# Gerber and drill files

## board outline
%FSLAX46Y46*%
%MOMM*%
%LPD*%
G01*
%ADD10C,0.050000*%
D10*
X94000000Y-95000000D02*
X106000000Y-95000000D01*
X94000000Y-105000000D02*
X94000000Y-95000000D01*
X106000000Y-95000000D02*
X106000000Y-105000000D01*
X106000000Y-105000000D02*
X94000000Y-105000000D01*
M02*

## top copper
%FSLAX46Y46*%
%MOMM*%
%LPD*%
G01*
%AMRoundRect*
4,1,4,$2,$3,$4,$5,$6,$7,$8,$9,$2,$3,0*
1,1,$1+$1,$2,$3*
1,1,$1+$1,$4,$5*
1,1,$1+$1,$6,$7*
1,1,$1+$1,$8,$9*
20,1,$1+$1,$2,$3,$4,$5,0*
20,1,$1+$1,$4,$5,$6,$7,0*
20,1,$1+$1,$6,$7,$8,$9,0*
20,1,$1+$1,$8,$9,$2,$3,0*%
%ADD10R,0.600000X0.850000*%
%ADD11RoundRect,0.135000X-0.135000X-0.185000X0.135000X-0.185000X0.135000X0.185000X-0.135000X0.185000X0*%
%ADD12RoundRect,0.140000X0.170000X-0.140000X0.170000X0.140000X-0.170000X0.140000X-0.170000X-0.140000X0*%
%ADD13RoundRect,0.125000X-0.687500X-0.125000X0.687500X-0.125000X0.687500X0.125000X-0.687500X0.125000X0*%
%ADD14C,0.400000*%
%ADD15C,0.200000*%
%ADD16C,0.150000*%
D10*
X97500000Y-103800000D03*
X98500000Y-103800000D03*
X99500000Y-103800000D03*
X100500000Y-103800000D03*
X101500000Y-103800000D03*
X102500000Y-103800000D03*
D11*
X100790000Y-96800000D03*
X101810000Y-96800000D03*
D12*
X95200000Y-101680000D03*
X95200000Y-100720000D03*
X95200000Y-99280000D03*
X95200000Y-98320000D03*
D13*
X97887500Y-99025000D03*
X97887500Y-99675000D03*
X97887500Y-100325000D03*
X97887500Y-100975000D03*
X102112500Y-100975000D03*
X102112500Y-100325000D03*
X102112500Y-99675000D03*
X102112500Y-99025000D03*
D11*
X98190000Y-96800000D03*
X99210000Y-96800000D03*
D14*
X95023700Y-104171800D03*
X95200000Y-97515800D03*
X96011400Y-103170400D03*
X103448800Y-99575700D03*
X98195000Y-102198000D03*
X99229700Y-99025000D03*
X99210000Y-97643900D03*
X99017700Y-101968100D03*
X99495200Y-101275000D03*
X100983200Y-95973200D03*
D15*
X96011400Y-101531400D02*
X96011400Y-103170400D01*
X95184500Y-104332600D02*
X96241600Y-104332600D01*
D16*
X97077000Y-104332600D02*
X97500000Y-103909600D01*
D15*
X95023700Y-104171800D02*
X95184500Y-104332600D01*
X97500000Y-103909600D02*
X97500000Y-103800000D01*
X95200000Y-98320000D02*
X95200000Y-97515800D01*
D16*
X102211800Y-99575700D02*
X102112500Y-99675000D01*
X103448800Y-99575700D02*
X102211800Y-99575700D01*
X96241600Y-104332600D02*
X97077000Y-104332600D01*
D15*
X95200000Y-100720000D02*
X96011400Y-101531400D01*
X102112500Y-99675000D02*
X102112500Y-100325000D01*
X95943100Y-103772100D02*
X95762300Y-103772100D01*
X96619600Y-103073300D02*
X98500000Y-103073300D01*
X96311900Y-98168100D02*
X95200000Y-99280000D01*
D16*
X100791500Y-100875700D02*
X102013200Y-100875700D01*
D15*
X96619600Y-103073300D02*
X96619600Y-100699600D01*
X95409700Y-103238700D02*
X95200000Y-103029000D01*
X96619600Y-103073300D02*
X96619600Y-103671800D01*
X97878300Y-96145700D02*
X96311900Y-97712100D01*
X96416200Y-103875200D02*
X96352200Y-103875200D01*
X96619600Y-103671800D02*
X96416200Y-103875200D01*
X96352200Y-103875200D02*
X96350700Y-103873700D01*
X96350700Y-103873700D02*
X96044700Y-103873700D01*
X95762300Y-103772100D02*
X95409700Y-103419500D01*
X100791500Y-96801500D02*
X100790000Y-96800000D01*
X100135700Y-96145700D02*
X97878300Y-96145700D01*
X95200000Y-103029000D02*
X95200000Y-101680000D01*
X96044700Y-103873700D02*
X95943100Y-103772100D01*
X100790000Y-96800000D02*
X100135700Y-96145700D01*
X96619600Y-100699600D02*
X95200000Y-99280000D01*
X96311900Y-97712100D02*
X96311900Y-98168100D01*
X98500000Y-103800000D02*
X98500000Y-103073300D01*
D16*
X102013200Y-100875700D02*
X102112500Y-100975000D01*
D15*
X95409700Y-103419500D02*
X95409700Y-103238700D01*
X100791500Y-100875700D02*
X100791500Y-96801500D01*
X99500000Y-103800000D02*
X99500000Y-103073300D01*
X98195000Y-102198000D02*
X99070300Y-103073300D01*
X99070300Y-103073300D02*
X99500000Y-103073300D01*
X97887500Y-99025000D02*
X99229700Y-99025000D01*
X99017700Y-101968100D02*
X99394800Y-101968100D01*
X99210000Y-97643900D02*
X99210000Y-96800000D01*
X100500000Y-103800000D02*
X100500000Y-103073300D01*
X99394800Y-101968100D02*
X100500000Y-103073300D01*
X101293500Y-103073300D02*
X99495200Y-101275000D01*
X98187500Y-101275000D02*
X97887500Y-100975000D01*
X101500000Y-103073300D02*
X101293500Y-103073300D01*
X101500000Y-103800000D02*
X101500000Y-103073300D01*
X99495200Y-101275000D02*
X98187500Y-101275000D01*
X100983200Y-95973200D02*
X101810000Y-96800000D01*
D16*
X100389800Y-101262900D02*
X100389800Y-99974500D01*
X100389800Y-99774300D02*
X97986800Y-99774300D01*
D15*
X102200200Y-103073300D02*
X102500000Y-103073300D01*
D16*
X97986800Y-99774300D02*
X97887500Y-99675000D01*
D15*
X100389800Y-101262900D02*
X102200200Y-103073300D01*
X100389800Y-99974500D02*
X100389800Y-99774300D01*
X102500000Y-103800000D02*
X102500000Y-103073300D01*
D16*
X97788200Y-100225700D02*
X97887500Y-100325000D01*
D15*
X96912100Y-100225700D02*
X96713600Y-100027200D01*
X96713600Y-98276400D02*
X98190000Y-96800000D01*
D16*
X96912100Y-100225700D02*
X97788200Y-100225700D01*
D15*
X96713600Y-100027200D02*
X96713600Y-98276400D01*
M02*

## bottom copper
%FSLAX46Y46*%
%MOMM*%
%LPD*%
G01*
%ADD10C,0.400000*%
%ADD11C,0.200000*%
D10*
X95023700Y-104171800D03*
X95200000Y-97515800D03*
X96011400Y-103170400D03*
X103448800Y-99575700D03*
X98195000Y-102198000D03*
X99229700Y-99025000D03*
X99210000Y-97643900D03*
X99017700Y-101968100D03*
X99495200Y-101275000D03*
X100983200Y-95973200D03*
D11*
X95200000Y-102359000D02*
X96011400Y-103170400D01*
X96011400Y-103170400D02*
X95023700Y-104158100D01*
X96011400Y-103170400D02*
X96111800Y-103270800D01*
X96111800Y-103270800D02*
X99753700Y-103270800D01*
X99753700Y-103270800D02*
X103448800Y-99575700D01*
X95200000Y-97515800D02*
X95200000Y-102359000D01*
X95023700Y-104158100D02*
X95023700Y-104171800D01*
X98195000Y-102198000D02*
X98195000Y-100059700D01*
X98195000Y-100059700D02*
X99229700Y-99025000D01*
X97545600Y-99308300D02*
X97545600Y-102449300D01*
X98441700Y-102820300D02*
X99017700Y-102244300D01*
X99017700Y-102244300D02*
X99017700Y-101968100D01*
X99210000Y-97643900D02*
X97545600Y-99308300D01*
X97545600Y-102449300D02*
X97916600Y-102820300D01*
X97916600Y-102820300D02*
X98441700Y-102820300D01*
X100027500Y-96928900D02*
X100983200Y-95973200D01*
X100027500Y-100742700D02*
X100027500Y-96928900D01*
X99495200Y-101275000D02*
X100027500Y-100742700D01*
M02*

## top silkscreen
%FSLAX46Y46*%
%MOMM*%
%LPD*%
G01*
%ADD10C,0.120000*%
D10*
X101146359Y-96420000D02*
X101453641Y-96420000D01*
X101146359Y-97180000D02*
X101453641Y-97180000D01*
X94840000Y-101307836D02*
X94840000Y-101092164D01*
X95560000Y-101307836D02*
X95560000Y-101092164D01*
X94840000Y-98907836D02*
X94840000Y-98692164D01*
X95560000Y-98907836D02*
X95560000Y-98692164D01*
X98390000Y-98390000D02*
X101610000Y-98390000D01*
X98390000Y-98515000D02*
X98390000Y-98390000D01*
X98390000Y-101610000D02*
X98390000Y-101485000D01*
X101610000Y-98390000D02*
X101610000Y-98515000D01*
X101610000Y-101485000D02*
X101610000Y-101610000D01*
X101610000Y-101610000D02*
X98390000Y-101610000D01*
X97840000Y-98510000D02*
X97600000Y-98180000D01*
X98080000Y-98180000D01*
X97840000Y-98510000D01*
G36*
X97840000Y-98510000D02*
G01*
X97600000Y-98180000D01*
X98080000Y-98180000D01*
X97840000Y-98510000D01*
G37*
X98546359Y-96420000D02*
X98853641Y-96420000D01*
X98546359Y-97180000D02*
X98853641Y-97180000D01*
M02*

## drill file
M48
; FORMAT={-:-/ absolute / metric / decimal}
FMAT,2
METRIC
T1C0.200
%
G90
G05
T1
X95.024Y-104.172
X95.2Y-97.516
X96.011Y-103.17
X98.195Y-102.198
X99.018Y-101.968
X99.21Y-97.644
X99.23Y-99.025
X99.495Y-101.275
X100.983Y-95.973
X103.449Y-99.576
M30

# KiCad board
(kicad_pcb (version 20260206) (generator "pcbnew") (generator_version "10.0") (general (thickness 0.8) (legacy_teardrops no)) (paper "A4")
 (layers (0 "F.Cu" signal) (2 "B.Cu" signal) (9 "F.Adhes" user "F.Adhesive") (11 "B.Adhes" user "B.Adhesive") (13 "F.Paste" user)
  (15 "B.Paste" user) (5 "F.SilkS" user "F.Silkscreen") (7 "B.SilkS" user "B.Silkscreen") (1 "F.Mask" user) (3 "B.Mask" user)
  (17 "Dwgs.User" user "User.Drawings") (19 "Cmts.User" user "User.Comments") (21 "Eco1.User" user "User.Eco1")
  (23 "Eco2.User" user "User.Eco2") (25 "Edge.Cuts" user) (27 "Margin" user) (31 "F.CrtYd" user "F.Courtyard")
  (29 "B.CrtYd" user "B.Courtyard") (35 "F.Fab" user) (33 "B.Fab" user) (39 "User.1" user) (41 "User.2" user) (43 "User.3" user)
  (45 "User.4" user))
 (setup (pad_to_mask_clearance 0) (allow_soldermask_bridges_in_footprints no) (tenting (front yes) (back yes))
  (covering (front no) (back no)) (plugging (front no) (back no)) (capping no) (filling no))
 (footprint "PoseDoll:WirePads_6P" (layer "F.Cu") (at 100 103.8)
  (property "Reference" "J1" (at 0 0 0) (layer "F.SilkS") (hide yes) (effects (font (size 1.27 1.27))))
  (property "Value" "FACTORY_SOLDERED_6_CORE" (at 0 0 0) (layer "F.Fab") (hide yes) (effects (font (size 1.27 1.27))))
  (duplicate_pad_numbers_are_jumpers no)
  (pad "1" smd rect (at -2.5 0) (size 0.6 0.85) (layers "F.Cu" "F.Mask") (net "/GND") (thermal_bridge_angle 45))
  (pad "2" smd rect (at -1.5 0) (size 0.6 0.85) (layers "F.Cu" "F.Mask") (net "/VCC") (thermal_bridge_angle 45))
  (pad "3" smd rect (at -0.5 0) (size 0.6 0.85) (layers "F.Cu" "F.Mask") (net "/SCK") (thermal_bridge_angle 45))
  (pad "4" smd rect (at 0.5 0) (size 0.6 0.85) (layers "F.Cu" "F.Mask") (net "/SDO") (thermal_bridge_angle 45))
  (pad "5" smd rect (at 1.5 0) (size 0.6 0.85) (layers "F.Cu" "F.Mask") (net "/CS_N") (thermal_bridge_angle 45))
  (pad "6" smd rect (at 2.5 0) (size 0.6 0.85) (layers "F.Cu" "F.Mask") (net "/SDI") (thermal_bridge_angle 45)))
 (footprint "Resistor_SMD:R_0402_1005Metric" (layer "F.Cu") (at 101.3 96.8)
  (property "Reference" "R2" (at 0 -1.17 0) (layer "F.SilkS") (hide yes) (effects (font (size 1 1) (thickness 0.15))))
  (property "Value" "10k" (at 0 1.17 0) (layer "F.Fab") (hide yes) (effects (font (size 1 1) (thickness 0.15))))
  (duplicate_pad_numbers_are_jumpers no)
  (fp_line (start -0.153641 -0.38) (end 0.153641 -0.38) (stroke (width 0.12) (type solid)) (layer "F.SilkS"))
  (fp_line (start -0.153641 0.38) (end 0.153641 0.38) (stroke (width 0.12) (type solid)) (layer "F.SilkS"))
  (pad "1" smd roundrect (at -0.51 0) (size 0.54 0.64) (layers "F.Cu" "F.Mask" "F.Paste") (roundrect_rratio 0.25) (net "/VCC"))
  (pad "2" smd roundrect (at 0.51 0) (size 0.54 0.64) (layers "F.Cu" "F.Mask" "F.Paste") (roundrect_rratio 0.25) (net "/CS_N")))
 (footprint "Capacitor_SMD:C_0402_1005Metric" (layer "F.Cu") (at 95.2 101.2 90)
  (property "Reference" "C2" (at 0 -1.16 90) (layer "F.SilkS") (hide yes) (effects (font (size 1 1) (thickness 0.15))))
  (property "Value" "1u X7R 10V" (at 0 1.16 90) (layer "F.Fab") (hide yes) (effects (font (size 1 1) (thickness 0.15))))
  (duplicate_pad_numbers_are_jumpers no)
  (fp_line (start -0.107836 -0.36) (end 0.107836 -0.36) (stroke (width 0.12) (type solid)) (layer "F.SilkS"))
  (fp_line (start -0.107836 0.36) (end 0.107836 0.36) (stroke (width 0.12) (type solid)) (layer "F.SilkS"))
  (pad "1" smd roundrect (at -0.48 0 90) (size 0.56 0.62) (layers "F.Cu" "F.Mask" "F.Paste") (roundrect_rratio 0.25) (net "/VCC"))
  (pad "2" smd roundrect (at 0.48 0 90) (size 0.56 0.62) (layers "F.Cu" "F.Mask" "F.Paste") (roundrect_rratio 0.25) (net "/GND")))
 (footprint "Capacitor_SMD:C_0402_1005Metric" (layer "F.Cu") (at 95.2 98.8 90)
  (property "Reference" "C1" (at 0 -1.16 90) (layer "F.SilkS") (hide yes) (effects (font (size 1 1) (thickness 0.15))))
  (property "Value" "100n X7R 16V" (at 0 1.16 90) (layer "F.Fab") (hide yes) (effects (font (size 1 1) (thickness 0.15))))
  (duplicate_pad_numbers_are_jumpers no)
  (fp_line (start -0.107836 -0.36) (end 0.107836 -0.36) (stroke (width 0.12) (type solid)) (layer "F.SilkS"))
  (fp_line (start -0.107836 0.36) (end 0.107836 0.36) (stroke (width 0.12) (type solid)) (layer "F.SilkS"))
  (pad "1" smd roundrect (at -0.48 0 90) (size 0.56 0.62) (layers "F.Cu" "F.Mask" "F.Paste") (roundrect_rratio 0.25) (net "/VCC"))
  (pad "2" smd roundrect (at 0.48 0 90) (size 0.56 0.62) (layers "F.Cu" "F.Mask" "F.Paste") (roundrect_rratio 0.25) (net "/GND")))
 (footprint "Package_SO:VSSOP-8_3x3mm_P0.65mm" (layer "F.Cu") (at 100 100)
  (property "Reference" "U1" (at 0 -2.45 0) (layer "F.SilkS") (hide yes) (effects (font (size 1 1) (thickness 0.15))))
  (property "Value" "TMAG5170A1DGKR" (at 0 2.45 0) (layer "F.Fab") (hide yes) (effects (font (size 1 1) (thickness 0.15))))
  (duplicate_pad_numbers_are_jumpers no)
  (fp_line (start -1.61 -1.61) (end 1.61 -1.61) (stroke (width 0.12) (type solid)) (layer "F.SilkS"))
  (fp_line (start -1.61 -1.485) (end -1.61 -1.61) (stroke (width 0.12) (type solid)) (layer "F.SilkS"))
  (fp_line (start -1.61 1.61) (end -1.61 1.485) (stroke (width 0.12) (type solid)) (layer "F.SilkS"))
  (fp_line (start 1.61 -1.61) (end 1.61 -1.485) (stroke (width 0.12) (type solid)) (layer "F.SilkS"))
  (fp_line (start 1.61 1.485) (end 1.61 1.61) (stroke (width 0.12) (type solid)) (layer "F.SilkS"))
  (fp_line (start 1.61 1.61) (end -1.61 1.61) (stroke (width 0.12) (type solid)) (layer "F.SilkS"))
  (fp_poly (pts (xy -2.16 -1.49) (xy -2.4 -1.82) (xy -1.92 -1.82)) (stroke (width 0.12) (type solid)) (fill yes) (layer "F.SilkS"))
  (pad "1" smd roundrect (at -2.1125 -0.975) (size 1.625 0.5) (layers "F.Cu" "F.Mask" "F.Paste") (roundrect_rratio 0.25) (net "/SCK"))
  (pad "2" smd roundrect (at -2.1125 -0.325) (size 1.625 0.5) (layers "F.Cu" "F.Mask" "F.Paste") (roundrect_rratio 0.25) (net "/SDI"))
  (pad "3" smd roundrect (at -2.1125 0.325) (size 1.625 0.5) (layers "F.Cu" "F.Mask" "F.Paste") (roundrect_rratio 0.25) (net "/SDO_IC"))
  (pad "4" smd roundrect (at -2.1125 0.975) (size 1.625 0.5) (layers "F.Cu" "F.Mask" "F.Paste") (roundrect_rratio 0.25) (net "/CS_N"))
  (pad "5" smd roundrect (at 2.1125 0.975) (size 1.625 0.5) (layers "F.Cu" "F.Mask" "F.Paste") (roundrect_rratio 0.25) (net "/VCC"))
  (pad "6" smd roundrect (at 2.1125 0.325) (size 1.625 0.5) (layers "F.Cu" "F.Mask" "F.Paste") (roundrect_rratio 0.25) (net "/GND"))
  (pad "7" smd roundrect (at 2.1125 -0.325) (size 1.625 0.5) (layers "F.Cu" "F.Mask" "F.Paste") (roundrect_rratio 0.25) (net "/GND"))
  (pad "8" smd roundrect (at 2.1125 -0.975) (size 1.625 0.5) (layers "F.Cu" "F.Mask" "F.Paste") (roundrect_rratio 0.25)
   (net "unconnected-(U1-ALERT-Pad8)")))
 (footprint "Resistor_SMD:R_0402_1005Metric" (layer "F.Cu") (at 98.7 96.8)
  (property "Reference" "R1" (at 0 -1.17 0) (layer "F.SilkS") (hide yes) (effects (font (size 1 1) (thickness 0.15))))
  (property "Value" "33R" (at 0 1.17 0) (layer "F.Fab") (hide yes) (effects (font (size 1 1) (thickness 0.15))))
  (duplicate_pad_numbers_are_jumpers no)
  (fp_line (start -0.153641 -0.38) (end 0.153641 -0.38) (stroke (width 0.12) (type solid)) (layer "F.SilkS"))
  (fp_line (start -0.153641 0.38) (end 0.153641 0.38) (stroke (width 0.12) (type solid)) (layer "F.SilkS"))
  (pad "1" smd roundrect (at -0.51 0) (size 0.54 0.64) (layers "F.Cu" "F.Mask" "F.Paste") (roundrect_rratio 0.25) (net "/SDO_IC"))
  (pad "2" smd roundrect (at 0.51 0) (size 0.54 0.64) (layers "F.Cu" "F.Mask" "F.Paste") (roundrect_rratio 0.25) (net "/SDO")))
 (gr_line (start 94 95) (end 106 95) (stroke (width 0.05) (type default)) (layer "Edge.Cuts"))
 (gr_line (start 94 105) (end 94 95) (stroke (width 0.05) (type default)) (layer "Edge.Cuts"))
 (gr_line (start 106 95) (end 106 105) (stroke (width 0.05) (type default)) (layer "Edge.Cuts"))
 (gr_line (start 106 105) (end 94 105) (stroke (width 0.05) (type default)) (layer "Edge.Cuts"))
 (segment (start 96.0114 101.5314) (end 96.0114 103.1704) (width 0.2) (layer "F.Cu") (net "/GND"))
 (segment (start 95.1845 104.3326) (end 96.2416 104.3326) (width 0.2) (layer "F.Cu") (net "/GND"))
 (segment (start 97.077 104.3326) (end 97.5 103.9096) (width 0.15) (layer "F.Cu") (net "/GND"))
 (segment (start 95.0237 104.1718) (end 95.1845 104.3326) (width 0.2) (layer "F.Cu") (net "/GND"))
 (segment (start 97.5 103.9096) (end 97.5 103.8) (width 0.2) (layer "F.Cu") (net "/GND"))
 (segment (start 95.2 98.32) (end 95.2 97.5158) (width 0.2) (layer "F.Cu") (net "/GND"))
 (segment (start 102.2118 99.5757) (end 102.1125 99.675) (width 0.15) (layer "F.Cu") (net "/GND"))
 (segment (start 103.4488 99.5757) (end 102.2118 99.5757) (width 0.15) (layer "F.Cu") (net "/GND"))
 (segment (start 96.2416 104.3326) (end 97.077 104.3326) (width 0.15) (layer "F.Cu") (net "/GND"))
 (segment (start 95.2 100.72) (end 96.0114 101.5314) (width 0.2) (layer "F.Cu") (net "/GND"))
 (segment (start 102.1125 99.675) (end 102.1125 100.325) (width 0.2) (layer "F.Cu") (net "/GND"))
 (via (at 95.0237 104.1718) (size 0.4) (drill 0.2) (layers "F.Cu" "B.Cu") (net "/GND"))
 (via (at 95.2 97.5158) (size 0.4) (drill 0.2) (layers "F.Cu" "B.Cu") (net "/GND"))
 (via (at 96.0114 103.1704) (size 0.4) (drill 0.2) (layers "F.Cu" "B.Cu") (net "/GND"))
 (via (at 103.4488 99.5757) (size 0.4) (drill 0.2) (layers "F.Cu" "B.Cu") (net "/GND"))
 (segment (start 95.2 102.359) (end 96.0114 103.1704) (width 0.2) (layer "B.Cu") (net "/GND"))
 (segment (start 96.0114 103.1704) (end 95.0237 104.1581) (width 0.2) (layer "B.Cu") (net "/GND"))
 (segment (start 96.0114 103.1704) (end 96.1118 103.2708) (width 0.2) (layer "B.Cu") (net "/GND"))
 (segment (start 96.1118 103.2708) (end 99.7537 103.2708) (width 0.2) (layer "B.Cu") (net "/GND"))
 (segment (start 99.7537 103.2708) (end 103.4488 99.5757) (width 0.2) (layer "B.Cu") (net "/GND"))
 (segment (start 95.2 97.5158) (end 95.2 102.359) (width 0.2) (layer "B.Cu") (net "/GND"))
 (segment (start 95.0237 104.1581) (end 95.0237 104.1718) (width 0.2) (layer "B.Cu") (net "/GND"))
 (segment (start 95.9431 103.7721) (end 95.7623 103.7721) (width 0.2) (layer "F.Cu") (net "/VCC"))
 (segment (start 96.6196 103.0733) (end 98.5 103.0733) (width 0.2) (layer "F.Cu") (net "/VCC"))
 (segment (start 96.3119 98.1681) (end 95.2 99.28) (width 0.2) (layer "F.Cu") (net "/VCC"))
 (segment (start 100.7915 100.8757) (end 102.0132 100.8757) (width 0.15) (layer "F.Cu") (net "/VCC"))
 (segment (start 96.6196 103.0733) (end 96.6196 100.6996) (width 0.2) (layer "F.Cu") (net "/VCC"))
 (segment (start 95.4097 103.2387) (end 95.2 103.029) (width 0.2) (layer "F.Cu") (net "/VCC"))
 (segment (start 96.6196 103.0733) (end 96.6196 103.6718) (width 0.2) (layer "F.Cu") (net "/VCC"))
 (segment (start 97.8783 96.1457) (end 96.3119 97.7121) (width 0.2) (layer "F.Cu") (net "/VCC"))
 (segment (start 96.4162 103.8752) (end 96.3522 103.8752) (width 0.2) (layer "F.Cu") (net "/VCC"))
 (segment (start 96.6196 103.6718) (end 96.4162 103.8752) (width 0.2) (layer "F.Cu") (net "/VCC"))
 (segment (start 96.3522 103.8752) (end 96.3507 103.8737) (width 0.2) (layer "F.Cu") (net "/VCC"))
 (segment (start 96.3507 103.8737) (end 96.0447 103.8737) (width 0.2) (layer "F.Cu") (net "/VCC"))
 (segment (start 95.7623 103.7721) (end 95.4097 103.4195) (width 0.2) (layer "F.Cu") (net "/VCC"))
 (segment (start 100.7915 96.8015) (end 100.79 96.8) (width 0.2) (layer "F.Cu") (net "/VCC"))
 (segment (start 100.1357 96.1457) (end 97.8783 96.1457) (width 0.2) (layer "F.Cu") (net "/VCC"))
 (segment (start 95.2 103.029) (end 95.2 101.68) (width 0.2) (layer "F.Cu") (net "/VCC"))
 (segment (start 96.0447 103.8737) (end 95.9431 103.7721) (width 0.2) (layer "F.Cu") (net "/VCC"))
 (segment (start 100.79 96.8) (end 100.1357 96.1457) (width 0.2) (layer "F.Cu") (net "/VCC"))
 (segment (start 96.6196 100.6996) (end 95.2 99.28) (width 0.2) (layer "F.Cu") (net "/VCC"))
 (segment (start 96.3119 97.7121) (end 96.3119 98.1681) (width 0.2) (layer "F.Cu") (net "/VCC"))
 (segment (start 98.5 103.8) (end 98.5 103.0733) (width 0.2) (layer "F.Cu") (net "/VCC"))
 (segment (start 102.0132 100.8757) (end 102.1125 100.975) (width 0.15) (layer "F.Cu") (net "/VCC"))
 (segment (start 95.4097 103.4195) (end 95.4097 103.2387) (width 0.2) (layer "F.Cu") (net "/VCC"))
 (segment (start 100.7915 100.8757) (end 100.7915 96.8015) (width 0.2) (layer "F.Cu") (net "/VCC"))
 (segment (start 99.5 103.8) (end 99.5 103.0733) (width 0.2) (layer "F.Cu") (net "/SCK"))
 (segment (start 98.195 102.198) (end 99.0703 103.0733) (width 0.2) (layer "F.Cu") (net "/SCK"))
 (segment (start 99.0703 103.0733) (end 99.5 103.0733) (width 0.2) (layer "F.Cu") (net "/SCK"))
 (segment (start 97.8875 99.025) (end 99.2297 99.025) (width 0.2) (layer "F.Cu") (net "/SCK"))
 (via (at 98.195 102.198) (size 0.4) (drill 0.2) (layers "F.Cu" "B.Cu") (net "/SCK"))
 (via (at 99.2297 99.025) (size 0.4) (drill 0.2) (layers "F.Cu" "B.Cu") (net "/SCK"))
 (segment (start 98.195 102.198) (end 98.195 100.0597) (width 0.2) (layer "B.Cu") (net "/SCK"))
 (segment (start 98.195 100.0597) (end 99.2297 99.025) (width 0.2) (layer "B.Cu") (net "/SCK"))
 (segment (start 99.0177 101.9681) (end 99.3948 101.9681) (width 0.2) (layer "F.Cu") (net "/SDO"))
 (segment (start 99.21 97.6439) (end 99.21 96.8) (width 0.2) (layer "F.Cu") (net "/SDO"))
 (segment (start 100.5 103.8) (end 100.5 103.0733) (width 0.2) (layer "F.Cu") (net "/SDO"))
 (segment (start 99.3948 101.9681) (end 100.5 103.0733) (width 0.2) (layer "F.Cu") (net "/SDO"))
 (via (at 99.21 97.6439) (size 0.4) (drill 0.2) (layers "F.Cu" "B.Cu") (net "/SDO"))
 (via (at 99.0177 101.9681) (size 0.4) (drill 0.2) (layers "F.Cu" "B.Cu") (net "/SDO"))
 (segment (start 97.5456 99.3083) (end 97.5456 102.4493) (width 0.2) (layer "B.Cu") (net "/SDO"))
 (segment (start 98.4417 102.8203) (end 99.0177 102.2443) (width 0.2) (layer "B.Cu") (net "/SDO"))
 (segment (start 99.0177 102.2443) (end 99.0177 101.9681) (width 0.2) (layer "B.Cu") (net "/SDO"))
 (segment (start 99.21 97.6439) (end 97.5456 99.3083) (width 0.2) (layer "B.Cu") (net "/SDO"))
 (segment (start 97.5456 102.4493) (end 97.9166 102.8203) (width 0.2) (layer "B.Cu") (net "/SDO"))
 (segment (start 97.9166 102.8203) (end 98.4417 102.8203) (width 0.2) (layer "B.Cu") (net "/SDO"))
 (segment (start 101.2935 103.0733) (end 99.4952 101.275) (width 0.2) (layer "F.Cu") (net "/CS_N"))
 (segment (start 98.1875 101.275) (end 97.8875 100.975) (width 0.2) (layer "F.Cu") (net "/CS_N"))
 (segment (start 101.5 103.0733) (end 101.2935 103.0733) (width 0.2) (layer "F.Cu") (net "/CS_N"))
 (segment (start 101.5 103.8) (end 101.5 103.0733) (width 0.2) (layer "F.Cu") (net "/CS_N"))
 (segment (start 99.4952 101.275) (end 98.1875 101.275) (width 0.2) (layer "F.Cu") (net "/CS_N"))
 (segment (start 100.9832 95.9732) (end 101.81 96.8) (width 0.2) (layer "F.Cu") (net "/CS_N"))
 (via (at 99.4952 101.275) (size 0.4) (drill 0.2) (layers "F.Cu" "B.Cu") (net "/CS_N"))
 (via (at 100.9832 95.9732) (size 0.4) (drill 0.2) (layers "F.Cu" "B.Cu") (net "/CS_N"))
 (segment (start 100.0275 96.9289) (end 100.9832 95.9732) (width 0.2) (layer "B.Cu") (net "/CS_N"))
 (segment (start 100.0275 100.7427) (end 100.0275 96.9289) (width 0.2) (layer "B.Cu") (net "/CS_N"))
 (segment (start 99.4952 101.275) (end 100.0275 100.7427) (width 0.2) (layer "B.Cu") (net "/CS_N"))
 (segment (start 100.3898 101.2629) (end 100.3898 99.9745) (width 0.15) (layer "F.Cu") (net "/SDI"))
 (segment (start 100.3898 99.7743) (end 97.9868 99.7743) (width 0.15) (layer "F.Cu") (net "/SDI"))
 (segment (start 102.2002 103.0733) (end 102.5 103.0733) (width 0.2) (layer "F.Cu") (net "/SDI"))
 (segment (start 97.9868 99.7743) (end 97.8875 99.675) (width 0.15) (layer "F.Cu") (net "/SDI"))
 (segment (start 100.3898 101.2629) (end 102.2002 103.0733) (width 0.2) (layer "F.Cu") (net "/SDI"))
 (segment (start 100.3898 99.9745) (end 100.3898 99.7743) (width 0.2) (layer "F.Cu") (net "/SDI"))
 (segment (start 102.5 103.8) (end 102.5 103.0733) (width 0.2) (layer "F.Cu") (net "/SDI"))
 (segment (start 97.7882 100.2257) (end 97.8875 100.325) (width 0.15) (layer "F.Cu") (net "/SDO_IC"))
 (segment (start 96.9121 100.2257) (end 96.7136 100.0272) (width 0.2) (layer "F.Cu") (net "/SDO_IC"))
 (segment (start 96.7136 98.2764) (end 98.19 96.8) (width 0.2) (layer "F.Cu") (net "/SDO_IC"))
 (segment (start 96.9121 100.2257) (end 97.7882 100.2257) (width 0.15) (layer "F.Cu") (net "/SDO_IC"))
 (segment (start 96.7136 100.0272) (end 96.7136 98.2764) (width 0.2) (layer "F.Cu") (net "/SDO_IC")))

